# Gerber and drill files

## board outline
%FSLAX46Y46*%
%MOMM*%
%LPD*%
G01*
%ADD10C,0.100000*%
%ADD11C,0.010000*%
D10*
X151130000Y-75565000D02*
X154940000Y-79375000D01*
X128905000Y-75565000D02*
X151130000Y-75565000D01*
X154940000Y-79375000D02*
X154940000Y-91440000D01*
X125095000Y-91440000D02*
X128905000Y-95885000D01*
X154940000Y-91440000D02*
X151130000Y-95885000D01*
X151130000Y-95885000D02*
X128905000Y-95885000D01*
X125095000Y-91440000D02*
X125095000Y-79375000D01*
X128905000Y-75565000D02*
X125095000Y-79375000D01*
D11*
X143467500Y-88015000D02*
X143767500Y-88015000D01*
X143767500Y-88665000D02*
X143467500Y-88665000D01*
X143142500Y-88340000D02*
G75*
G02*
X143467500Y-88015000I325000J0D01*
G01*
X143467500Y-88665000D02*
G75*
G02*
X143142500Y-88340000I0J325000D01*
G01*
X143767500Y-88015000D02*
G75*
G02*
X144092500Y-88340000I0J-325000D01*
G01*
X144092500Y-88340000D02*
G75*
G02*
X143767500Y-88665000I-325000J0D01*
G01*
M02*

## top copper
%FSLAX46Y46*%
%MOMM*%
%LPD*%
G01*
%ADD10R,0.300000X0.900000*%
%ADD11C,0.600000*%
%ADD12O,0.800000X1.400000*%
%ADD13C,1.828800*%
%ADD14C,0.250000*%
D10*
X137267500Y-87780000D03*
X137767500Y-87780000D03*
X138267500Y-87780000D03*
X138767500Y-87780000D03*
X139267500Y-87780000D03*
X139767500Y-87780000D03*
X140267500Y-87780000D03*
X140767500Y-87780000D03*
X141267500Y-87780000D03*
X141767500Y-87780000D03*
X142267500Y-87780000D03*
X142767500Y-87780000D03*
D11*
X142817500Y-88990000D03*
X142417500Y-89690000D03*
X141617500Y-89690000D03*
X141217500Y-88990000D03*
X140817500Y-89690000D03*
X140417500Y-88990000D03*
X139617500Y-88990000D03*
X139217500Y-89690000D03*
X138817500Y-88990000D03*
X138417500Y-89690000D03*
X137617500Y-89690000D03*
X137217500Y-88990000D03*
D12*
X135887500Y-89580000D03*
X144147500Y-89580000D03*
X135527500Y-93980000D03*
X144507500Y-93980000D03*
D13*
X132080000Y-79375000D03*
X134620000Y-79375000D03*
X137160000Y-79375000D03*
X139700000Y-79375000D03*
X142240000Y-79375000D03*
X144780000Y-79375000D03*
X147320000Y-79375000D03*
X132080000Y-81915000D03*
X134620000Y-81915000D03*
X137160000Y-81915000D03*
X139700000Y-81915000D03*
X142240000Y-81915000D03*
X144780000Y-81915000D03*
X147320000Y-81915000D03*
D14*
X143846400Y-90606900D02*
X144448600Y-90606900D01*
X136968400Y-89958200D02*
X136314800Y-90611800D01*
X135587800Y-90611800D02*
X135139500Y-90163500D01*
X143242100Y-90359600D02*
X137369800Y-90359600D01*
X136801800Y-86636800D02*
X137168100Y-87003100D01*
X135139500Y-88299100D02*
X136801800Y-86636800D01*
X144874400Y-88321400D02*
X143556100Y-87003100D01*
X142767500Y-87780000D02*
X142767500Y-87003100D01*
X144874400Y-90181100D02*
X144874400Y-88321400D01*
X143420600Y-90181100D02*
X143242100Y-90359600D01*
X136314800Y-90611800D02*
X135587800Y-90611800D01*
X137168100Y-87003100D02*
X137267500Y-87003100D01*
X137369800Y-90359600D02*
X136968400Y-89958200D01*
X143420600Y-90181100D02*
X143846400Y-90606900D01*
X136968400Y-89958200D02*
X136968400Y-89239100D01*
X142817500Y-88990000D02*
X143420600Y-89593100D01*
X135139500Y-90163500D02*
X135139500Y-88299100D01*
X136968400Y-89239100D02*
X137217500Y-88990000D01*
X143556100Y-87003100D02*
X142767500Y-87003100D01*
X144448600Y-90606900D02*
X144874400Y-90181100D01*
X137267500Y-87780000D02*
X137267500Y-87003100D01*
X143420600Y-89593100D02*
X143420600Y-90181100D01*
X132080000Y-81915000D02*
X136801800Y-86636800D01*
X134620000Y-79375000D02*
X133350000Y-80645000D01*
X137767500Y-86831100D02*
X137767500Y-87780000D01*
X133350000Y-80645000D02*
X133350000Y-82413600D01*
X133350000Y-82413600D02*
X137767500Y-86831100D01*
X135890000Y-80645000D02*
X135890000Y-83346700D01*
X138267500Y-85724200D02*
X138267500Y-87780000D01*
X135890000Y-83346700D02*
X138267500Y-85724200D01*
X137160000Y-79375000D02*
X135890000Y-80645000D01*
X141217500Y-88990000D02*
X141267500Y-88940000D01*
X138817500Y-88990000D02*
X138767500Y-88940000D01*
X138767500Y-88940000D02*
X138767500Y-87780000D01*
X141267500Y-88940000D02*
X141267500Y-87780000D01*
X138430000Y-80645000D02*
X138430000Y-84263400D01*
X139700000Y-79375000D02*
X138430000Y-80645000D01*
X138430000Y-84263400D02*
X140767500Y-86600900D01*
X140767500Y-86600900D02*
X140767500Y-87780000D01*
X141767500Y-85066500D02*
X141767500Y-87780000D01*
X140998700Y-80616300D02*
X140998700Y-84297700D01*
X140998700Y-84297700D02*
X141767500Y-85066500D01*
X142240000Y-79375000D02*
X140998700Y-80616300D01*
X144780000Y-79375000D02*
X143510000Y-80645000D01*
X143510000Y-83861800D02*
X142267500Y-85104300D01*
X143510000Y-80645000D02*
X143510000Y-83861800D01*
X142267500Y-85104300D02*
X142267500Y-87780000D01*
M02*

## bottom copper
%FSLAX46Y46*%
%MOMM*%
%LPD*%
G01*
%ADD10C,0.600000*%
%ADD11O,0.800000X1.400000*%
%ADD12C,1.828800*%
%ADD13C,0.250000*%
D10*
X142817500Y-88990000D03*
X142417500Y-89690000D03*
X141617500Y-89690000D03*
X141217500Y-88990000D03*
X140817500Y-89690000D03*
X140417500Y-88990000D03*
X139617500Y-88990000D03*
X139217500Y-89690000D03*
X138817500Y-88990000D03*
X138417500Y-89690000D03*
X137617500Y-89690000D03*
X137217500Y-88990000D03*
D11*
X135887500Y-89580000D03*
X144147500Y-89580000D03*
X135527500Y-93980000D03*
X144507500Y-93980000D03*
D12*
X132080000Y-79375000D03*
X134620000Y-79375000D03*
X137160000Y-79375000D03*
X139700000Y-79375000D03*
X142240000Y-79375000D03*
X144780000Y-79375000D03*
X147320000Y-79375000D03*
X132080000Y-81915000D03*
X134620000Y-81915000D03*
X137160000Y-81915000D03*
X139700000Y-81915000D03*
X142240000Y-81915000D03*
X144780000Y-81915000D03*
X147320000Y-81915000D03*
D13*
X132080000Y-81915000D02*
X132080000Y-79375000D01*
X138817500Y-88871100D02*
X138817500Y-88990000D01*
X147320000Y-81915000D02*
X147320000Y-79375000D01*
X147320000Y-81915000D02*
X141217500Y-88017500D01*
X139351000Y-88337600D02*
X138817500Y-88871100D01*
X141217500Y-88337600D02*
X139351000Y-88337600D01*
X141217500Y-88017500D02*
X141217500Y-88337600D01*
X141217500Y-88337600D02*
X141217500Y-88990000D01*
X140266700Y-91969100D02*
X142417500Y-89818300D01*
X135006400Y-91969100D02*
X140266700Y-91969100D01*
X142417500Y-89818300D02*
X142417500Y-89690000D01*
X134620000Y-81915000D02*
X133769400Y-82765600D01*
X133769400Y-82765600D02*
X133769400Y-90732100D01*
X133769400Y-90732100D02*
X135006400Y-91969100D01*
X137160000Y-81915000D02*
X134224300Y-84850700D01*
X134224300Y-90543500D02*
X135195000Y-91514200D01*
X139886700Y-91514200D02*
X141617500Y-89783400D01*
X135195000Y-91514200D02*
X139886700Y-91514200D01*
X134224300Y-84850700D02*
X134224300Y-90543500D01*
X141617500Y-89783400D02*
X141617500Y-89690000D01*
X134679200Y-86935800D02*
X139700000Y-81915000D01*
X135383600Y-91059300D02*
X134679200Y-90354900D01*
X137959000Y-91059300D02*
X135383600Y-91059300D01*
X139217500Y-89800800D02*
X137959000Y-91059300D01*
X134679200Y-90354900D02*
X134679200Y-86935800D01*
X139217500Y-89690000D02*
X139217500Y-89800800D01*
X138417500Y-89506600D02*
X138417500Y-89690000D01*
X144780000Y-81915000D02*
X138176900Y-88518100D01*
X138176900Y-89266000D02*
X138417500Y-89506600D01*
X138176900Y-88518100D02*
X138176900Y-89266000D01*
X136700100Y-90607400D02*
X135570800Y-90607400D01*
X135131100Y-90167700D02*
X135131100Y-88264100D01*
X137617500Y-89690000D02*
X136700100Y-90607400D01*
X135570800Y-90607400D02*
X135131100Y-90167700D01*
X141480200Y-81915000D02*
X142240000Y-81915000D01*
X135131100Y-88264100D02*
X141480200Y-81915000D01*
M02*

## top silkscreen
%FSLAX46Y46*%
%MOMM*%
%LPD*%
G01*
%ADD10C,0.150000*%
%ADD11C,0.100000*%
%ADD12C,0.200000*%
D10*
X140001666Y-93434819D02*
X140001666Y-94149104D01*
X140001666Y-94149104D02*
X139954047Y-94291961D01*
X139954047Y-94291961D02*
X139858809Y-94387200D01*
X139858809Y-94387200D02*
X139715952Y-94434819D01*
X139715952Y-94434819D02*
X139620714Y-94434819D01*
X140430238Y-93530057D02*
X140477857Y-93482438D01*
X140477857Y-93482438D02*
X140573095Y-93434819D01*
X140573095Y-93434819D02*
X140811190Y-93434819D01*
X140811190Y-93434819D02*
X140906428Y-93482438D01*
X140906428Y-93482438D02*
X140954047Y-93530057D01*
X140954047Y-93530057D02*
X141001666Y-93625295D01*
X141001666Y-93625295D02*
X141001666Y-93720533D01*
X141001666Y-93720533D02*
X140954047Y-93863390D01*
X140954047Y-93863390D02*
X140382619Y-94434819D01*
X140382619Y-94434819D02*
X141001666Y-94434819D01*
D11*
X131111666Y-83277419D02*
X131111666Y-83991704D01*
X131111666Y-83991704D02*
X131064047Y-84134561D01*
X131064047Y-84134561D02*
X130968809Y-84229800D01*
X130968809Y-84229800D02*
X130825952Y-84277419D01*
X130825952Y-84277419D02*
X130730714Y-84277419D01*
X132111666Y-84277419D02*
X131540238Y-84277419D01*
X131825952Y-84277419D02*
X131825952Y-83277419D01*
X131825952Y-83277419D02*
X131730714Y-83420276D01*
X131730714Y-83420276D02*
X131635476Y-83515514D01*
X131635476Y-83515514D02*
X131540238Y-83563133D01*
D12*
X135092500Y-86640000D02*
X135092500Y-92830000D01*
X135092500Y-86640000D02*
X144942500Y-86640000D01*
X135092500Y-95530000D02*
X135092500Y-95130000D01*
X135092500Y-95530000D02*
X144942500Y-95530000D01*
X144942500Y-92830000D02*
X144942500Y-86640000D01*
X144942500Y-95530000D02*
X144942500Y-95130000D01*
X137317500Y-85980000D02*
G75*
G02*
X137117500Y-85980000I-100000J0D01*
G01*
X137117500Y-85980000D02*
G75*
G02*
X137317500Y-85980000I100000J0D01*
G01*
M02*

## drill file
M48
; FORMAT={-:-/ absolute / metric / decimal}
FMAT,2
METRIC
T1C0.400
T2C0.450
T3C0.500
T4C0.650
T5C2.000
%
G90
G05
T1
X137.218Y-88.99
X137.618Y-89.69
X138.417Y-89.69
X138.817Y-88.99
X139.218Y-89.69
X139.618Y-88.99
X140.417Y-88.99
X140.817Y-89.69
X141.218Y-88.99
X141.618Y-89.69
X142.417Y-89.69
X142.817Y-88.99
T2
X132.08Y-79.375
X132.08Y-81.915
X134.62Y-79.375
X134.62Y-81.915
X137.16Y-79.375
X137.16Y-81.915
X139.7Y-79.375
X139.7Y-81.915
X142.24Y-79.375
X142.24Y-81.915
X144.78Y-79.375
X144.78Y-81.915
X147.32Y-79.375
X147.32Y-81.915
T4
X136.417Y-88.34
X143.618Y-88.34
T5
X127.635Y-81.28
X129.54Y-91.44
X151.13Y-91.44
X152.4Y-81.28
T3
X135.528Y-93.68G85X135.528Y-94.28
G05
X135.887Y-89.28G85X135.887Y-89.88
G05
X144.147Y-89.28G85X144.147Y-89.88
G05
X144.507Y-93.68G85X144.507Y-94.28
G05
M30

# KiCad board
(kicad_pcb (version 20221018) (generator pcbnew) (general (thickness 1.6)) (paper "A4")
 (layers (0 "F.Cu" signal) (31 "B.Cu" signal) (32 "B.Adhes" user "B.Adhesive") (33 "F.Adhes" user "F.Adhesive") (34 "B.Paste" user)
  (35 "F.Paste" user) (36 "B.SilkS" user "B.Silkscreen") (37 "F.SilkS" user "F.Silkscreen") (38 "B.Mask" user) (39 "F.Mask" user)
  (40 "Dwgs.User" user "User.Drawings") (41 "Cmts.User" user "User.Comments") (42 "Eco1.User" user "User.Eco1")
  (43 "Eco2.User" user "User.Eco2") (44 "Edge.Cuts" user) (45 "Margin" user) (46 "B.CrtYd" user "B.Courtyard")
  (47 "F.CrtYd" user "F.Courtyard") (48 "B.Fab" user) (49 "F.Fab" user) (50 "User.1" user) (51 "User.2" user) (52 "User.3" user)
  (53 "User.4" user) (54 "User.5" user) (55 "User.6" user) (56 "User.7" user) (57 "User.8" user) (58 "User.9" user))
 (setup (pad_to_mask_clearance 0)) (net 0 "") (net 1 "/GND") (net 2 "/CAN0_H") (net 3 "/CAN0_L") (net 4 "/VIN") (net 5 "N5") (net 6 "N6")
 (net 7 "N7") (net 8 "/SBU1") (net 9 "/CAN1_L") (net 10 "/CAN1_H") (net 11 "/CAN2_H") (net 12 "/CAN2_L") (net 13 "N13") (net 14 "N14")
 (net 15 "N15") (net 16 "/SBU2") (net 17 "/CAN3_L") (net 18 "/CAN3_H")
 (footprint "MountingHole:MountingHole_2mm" (layer "F.Cu") (at 152.4 81.28)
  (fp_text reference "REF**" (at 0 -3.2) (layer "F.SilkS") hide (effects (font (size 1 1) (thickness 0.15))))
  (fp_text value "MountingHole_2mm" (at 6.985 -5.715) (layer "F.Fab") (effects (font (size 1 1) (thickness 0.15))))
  (pad "" np_thru_hole circle (at 0 0) (size 2 2) (drill 2) (layers "*.Cu" "*.Mask")))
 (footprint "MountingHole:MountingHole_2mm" (layer "F.Cu") (at 151.13 91.44)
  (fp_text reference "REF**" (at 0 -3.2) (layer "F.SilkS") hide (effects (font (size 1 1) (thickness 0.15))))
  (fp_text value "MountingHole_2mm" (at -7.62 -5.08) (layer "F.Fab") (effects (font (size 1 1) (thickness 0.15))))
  (pad "" np_thru_hole circle (at 0 0) (size 2 2) (drill 2) (layers "F&B.Cu" "*.Mask")))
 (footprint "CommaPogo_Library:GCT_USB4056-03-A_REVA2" (layer "F.Cu") (at 140.0175 93.98)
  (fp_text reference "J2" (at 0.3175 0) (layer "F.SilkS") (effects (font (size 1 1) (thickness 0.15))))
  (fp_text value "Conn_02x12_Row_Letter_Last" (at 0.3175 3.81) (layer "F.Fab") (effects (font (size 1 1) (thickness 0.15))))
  (fp_line (start -4.925 -7.34) (end -4.925 -1.15) (stroke (width 0.2) (type solid)) (layer "F.SilkS"))
  (fp_line (start -4.925 -7.34) (end 4.925 -7.34) (stroke (width 0.2) (type solid)) (layer "F.SilkS"))
  (fp_line (start -4.925 1.55) (end -4.925 1.15) (stroke (width 0.2) (type solid)) (layer "F.SilkS"))
  (fp_line (start -4.925 1.55) (end 4.925 1.55) (stroke (width 0.2) (type solid)) (layer "F.SilkS"))
  (fp_line (start 4.925 -1.15) (end 4.925 -7.34) (stroke (width 0.2) (type solid)) (layer "F.SilkS"))
  (fp_line (start 4.925 1.55) (end 4.925 1.15) (stroke (width 0.2) (type solid)) (layer "F.SilkS"))
  (fp_circle (center -2.8 -8) (end -2.7 -8) (stroke (width 0.2) (type solid)) (fill none) (layer "F.SilkS"))
  (fp_line (start 3.45 -5.965) (end 3.75 -5.965) (stroke (width 0.01) (type solid)) (layer "Edge.Cuts"))
  (fp_line (start 3.75 -5.315) (end 3.45 -5.315) (stroke (width 0.01) (type solid)) (layer "Edge.Cuts"))
  (fp_arc (start 3.125 -5.64) (mid 3.22019 -5.86981) (end 3.45 -5.965) (stroke (width 0.01) (type solid)) (layer "Edge.Cuts"))
  (fp_arc (start 3.45 -5.315) (mid 3.22019 -5.41019) (end 3.125 -5.64) (stroke (width 0.01) (type solid)) (layer "Edge.Cuts"))
  (fp_arc (start 3.75 -5.965) (mid 3.97981 -5.86981) (end 4.075 -5.64) (stroke (width 0.01) (type solid)) (layer "Edge.Cuts"))
  (fp_arc (start 4.075 -5.64) (mid 3.97981 -5.41019) (end 3.75 -5.315) (stroke (width 0.01) (type solid)) (layer "Edge.Cuts"))
  (pad "" np_thru_hole circle (at -3.6 -5.64) (size 0.65 0.65) (drill 0.65) (layers "*.Cu" "*.Mask"))
  (pad "" np_thru_hole circle (at 3.6 -5.64) (size 0.65 0.65) (drill 0.65) (layers "*.Cu" "*.Mask"))
  (pad "A1" smd rect (at -2.75 -6.2) (size 0.3 0.9) (layers "F.Cu" "F.Paste" "F.Mask") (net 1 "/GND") (solder_mask_margin 0.102))
  (pad "A2" smd rect (at -2.25 -6.2) (size 0.3 0.9) (layers "F.Cu" "F.Paste" "F.Mask") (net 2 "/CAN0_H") (solder_mask_margin 0.102))
  (pad "A3" smd rect (at -1.75 -6.2) (size 0.3 0.9) (layers "F.Cu" "F.Paste" "F.Mask") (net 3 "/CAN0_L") (solder_mask_margin 0.102))
  (pad "A4" smd rect (at -1.25 -6.2) (size 0.3 0.9) (layers "F.Cu" "F.Paste" "F.Mask") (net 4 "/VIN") (solder_mask_margin 0.102))
  (pad "A5" smd rect (at -0.75 -6.2) (size 0.3 0.9) (layers "F.Cu" "F.Paste" "F.Mask") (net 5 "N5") (solder_mask_margin 0.102))
  (pad "A6" smd rect (at -0.25 -6.2) (size 0.3 0.9) (layers "F.Cu" "F.Paste" "F.Mask") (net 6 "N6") (solder_mask_margin 0.102))
  (pad "A7" smd rect (at 0.25 -6.2) (size 0.3 0.9) (layers "F.Cu" "F.Paste" "F.Mask") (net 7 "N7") (solder_mask_margin 0.102))
  (pad "A8" smd rect (at 0.75 -6.2) (size 0.3 0.9) (layers "F.Cu" "F.Paste" "F.Mask") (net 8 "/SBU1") (solder_mask_margin 0.102))
  (pad "A9" smd rect (at 1.25 -6.2) (size 0.3 0.9) (layers "F.Cu" "F.Paste" "F.Mask") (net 4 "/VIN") (solder_mask_margin 0.102))
  (pad "A10" smd rect (at 1.75 -6.2) (size 0.3 0.9) (layers "F.Cu" "F.Paste" "F.Mask") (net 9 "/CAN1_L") (solder_mask_margin 0.102))
  (pad "A11" smd rect (at 2.25 -6.2) (size 0.3 0.9) (layers "F.Cu" "F.Paste" "F.Mask") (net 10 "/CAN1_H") (solder_mask_margin 0.102))
  (pad "A12" smd rect (at 2.75 -6.2) (size 0.3 0.9) (layers "F.Cu" "F.Paste" "F.Mask") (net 1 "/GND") (solder_mask_margin 0.102))
  (pad "B1" thru_hole circle (at 2.8 -4.99) (size 0.6 0.6) (drill 0.4) (layers "*.Cu" "*.Mask") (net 1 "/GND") (solder_mask_margin 0.102))
  (pad "B2" thru_hole circle (at 2.4 -4.29) (size 0.6 0.6) (drill 0.4) (layers "*.Cu" "*.Mask") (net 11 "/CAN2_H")
   (solder_mask_margin 0.102))
  (pad "B3" thru_hole circle (at 1.6 -4.29) (size 0.6 0.6) (drill 0.4) (layers "*.Cu" "*.Mask") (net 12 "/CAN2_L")
   (solder_mask_margin 0.102))
  (pad "B4" thru_hole circle (at 1.2 -4.99) (size 0.6 0.6) (drill 0.4) (layers "*.Cu" "*.Mask") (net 4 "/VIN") (solder_mask_margin 0.102))
  (pad "B5" thru_hole circle (at 0.8 -4.29) (size 0.6 0.6) (drill 0.4) (layers "*.Cu" "*.Mask") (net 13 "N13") (solder_mask_margin 0.102))
  (pad "B6" thru_hole circle (at 0.4 -4.99) (size 0.6 0.6) (drill 0.4) (layers "*.Cu" "*.Mask") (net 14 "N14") (solder_mask_margin 0.102))
  (pad "B7" thru_hole circle (at -0.4 -4.99) (size 0.6 0.6) (drill 0.4) (layers "*.Cu" "*.Mask") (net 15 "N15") (solder_mask_margin 0.102))
  (pad "B8" thru_hole circle (at -0.8 -4.29) (size 0.6 0.6) (drill 0.4) (layers "*.Cu" "*.Mask") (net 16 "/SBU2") (solder_mask_margin 0.102))
  (pad "B9" thru_hole circle (at -1.2 -4.99) (size 0.6 0.6) (drill 0.4) (layers "*.Cu" "*.Mask") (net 4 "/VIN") (solder_mask_margin 0.102))
  (pad "B10" thru_hole circle (at -1.6 -4.29) (size 0.6 0.6) (drill 0.4) (layers "*.Cu" "*.Mask") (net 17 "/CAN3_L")
   (solder_mask_margin 0.102))
  (pad "B11" thru_hole circle (at -2.4 -4.29) (size 0.6 0.6) (drill 0.4) (layers "*.Cu" "*.Mask") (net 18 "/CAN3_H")
   (solder_mask_margin 0.102))
  (pad "B12" thru_hole circle (at -2.8 -4.99) (size 0.6 0.6) (drill 0.4) (layers "*.Cu" "*.Mask") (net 1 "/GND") (solder_mask_margin 0.102))
  (pad "S1" thru_hole oval (at -4.13 -4.4) (size 0.8 1.4) (drill oval 0.5 1.1) (layers "*.Cu" "*.Mask") (solder_mask_margin 0.102))
  (pad "S2" thru_hole oval (at 4.13 -4.4) (size 0.8 1.4) (drill oval 0.5 1.1) (layers "*.Cu" "*.Mask") (solder_mask_margin 0.102))
  (pad "S3" thru_hole oval (at -4.49 0) (size 0.8 1.4) (drill oval 0.5 1.1) (layers "*.Cu" "*.Mask") (solder_mask_margin 0.102))
  (pad "S4" thru_hole oval (at 4.49 0) (size 0.8 1.4) (drill oval 0.5 1.1) (layers "*.Cu" "*.Mask") (solder_mask_margin 0.102)))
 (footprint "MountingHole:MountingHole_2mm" (layer "F.Cu") (at 127.635 81.28)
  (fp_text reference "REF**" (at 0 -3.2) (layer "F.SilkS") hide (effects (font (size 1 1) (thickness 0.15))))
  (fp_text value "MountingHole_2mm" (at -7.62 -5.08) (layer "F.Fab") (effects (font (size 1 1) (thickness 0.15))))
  (pad "" np_thru_hole circle (at 0 0) (size 2 2) (drill 2) (layers "*.Cu" "*.Mask")))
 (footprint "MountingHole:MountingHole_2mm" (layer "F.Cu") (at 129.54 91.44)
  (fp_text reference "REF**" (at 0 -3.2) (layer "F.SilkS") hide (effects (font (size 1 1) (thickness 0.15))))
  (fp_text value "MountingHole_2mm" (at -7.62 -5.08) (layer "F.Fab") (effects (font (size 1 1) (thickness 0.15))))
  (pad "" np_thru_hole circle (at 0 0) (size 2 2) (drill 2) (layers "F&B.Cu" "*.Mask")))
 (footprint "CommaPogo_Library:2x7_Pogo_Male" (layer "F.Cu") (at 139.7 83.82)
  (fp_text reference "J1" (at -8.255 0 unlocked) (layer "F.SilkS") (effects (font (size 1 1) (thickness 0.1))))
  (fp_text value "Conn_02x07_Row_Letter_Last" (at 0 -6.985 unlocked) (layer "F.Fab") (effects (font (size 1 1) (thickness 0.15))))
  (pad "1" thru_hole circle (at -7.62 -4.445) (size 1.8288 1.8288) (drill 0.45) (layers "*.Cu" "*.Mask") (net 1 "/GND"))
  (pad "2" thru_hole circle (at -5.08 -4.445) (size 1.8288 1.8288) (drill 0.45) (layers "*.Cu" "*.Mask") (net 2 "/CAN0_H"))
  (pad "3" thru_hole circle (at -2.54 -4.445) (size 1.8288 1.8288) (drill 0.45) (layers "*.Cu" "*.Mask") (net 3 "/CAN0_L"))
  (pad "4" thru_hole circle (at 0 -4.445) (size 1.8288 1.8288) (drill 0.45) (layers "*.Cu" "*.Mask") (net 8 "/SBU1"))
  (pad "5" thru_hole circle (at 2.54 -4.445) (size 1.8288 1.8288) (drill 0.45) (layers "*.Cu" "*.Mask") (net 9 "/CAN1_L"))
  (pad "6" thru_hole circle (at 5.08 -4.445) (size 1.8288 1.8288) (drill 0.45) (layers "*.Cu" "*.Mask") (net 10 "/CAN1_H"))
  (pad "7" thru_hole circle (at 7.62 -4.445) (size 1.8288 1.8288) (drill 0.45) (layers "*.Cu" "*.Mask") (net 4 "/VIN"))
  (pad "8" thru_hole circle (at -7.62 -1.905) (size 1.8288 1.8288) (drill 0.45) (layers "*.Cu" "*.Mask") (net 1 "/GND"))
  (pad "9" thru_hole circle (at -5.08 -1.905) (size 1.8288 1.8288) (drill 0.45) (layers "*.Cu" "*.Mask") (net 11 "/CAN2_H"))
  (pad "10" thru_hole circle (at -2.54 -1.905) (size 1.8288 1.8288) (drill 0.45) (layers "*.Cu" "*.Mask") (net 12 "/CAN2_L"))
  (pad "11" thru_hole circle (at 0 -1.905) (size 1.8288 1.8288) (drill 0.45) (layers "*.Cu" "*.Mask") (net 16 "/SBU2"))
  (pad "12" thru_hole circle (at 2.54 -1.905) (size 1.8288 1.8288) (drill 0.45) (layers "*.Cu" "*.Mask") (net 18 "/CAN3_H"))
  (pad "13" thru_hole circle (at 5.08 -1.905) (size 1.8288 1.8288) (drill 0.45) (layers "*.Cu" "*.Mask") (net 17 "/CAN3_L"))
  (pad "14" thru_hole circle (at 7.62 -1.905) (size 1.8288 1.8288) (drill 0.45) (layers "*.Cu" "*.Mask") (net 4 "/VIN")))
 (gr_line (start 151.13 75.565) (end 154.94 79.375) (stroke (width 0.1) (type default)) (layer "Edge.Cuts"))
 (gr_line (start 128.905 75.565) (end 151.13 75.565) (stroke (width 0.1) (type default)) (layer "Edge.Cuts"))
 (gr_line (start 154.94 79.375) (end 154.94 91.44) (stroke (width 0.1) (type default)) (layer "Edge.Cuts"))
 (gr_line (start 125.095 91.44) (end 128.905 95.885) (stroke (width 0.1) (type default)) (layer "Edge.Cuts"))
 (gr_line (start 154.94 91.44) (end 151.13 95.885) (stroke (width 0.1) (type default)) (layer "Edge.Cuts"))
 (gr_line (start 151.13 95.885) (end 128.905 95.885) (stroke (width 0.1) (type default)) (layer "Edge.Cuts"))
 (gr_line (start 125.095 91.44) (end 125.095 79.375) (stroke (width 0.1) (type default)) (layer "Edge.Cuts"))
 (gr_line (start 128.905 75.565) (end 125.095 79.375) (stroke (width 0.1) (type default)) (layer "Edge.Cuts"))
 (segment (start 143.8464 90.6069) (end 144.4486 90.6069) (width 0.25) (layer "F.Cu") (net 1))
 (segment (start 136.9684 89.9582) (end 136.3148 90.6118) (width 0.25) (layer "F.Cu") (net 1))
 (segment (start 135.5878 90.6118) (end 135.1395 90.1635) (width 0.25) (layer "F.Cu") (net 1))
 (segment (start 143.2421 90.3596) (end 137.3698 90.3596) (width 0.25) (layer "F.Cu") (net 1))
 (segment (start 136.8018 86.6368) (end 137.1681 87.0031) (width 0.25) (layer "F.Cu") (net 1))
 (segment (start 135.1395 88.2991) (end 136.8018 86.6368) (width 0.25) (layer "F.Cu") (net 1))
 (segment (start 144.8744 88.3214) (end 143.5561 87.0031) (width 0.25) (layer "F.Cu") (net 1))
 (segment (start 142.7675 87.78) (end 142.7675 87.0031) (width 0.25) (layer "F.Cu") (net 1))
 (segment (start 144.8744 90.1811) (end 144.8744 88.3214) (width 0.25) (layer "F.Cu") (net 1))
 (segment (start 143.4206 90.1811) (end 143.2421 90.3596) (width 0.25) (layer "F.Cu") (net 1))
 (segment (start 136.3148 90.6118) (end 135.5878 90.6118) (width 0.25) (layer "F.Cu") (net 1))
 (segment (start 137.1681 87.0031) (end 137.2675 87.0031) (width 0.25) (layer "F.Cu") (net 1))
 (segment (start 137.3698 90.3596) (end 136.9684 89.9582) (width 0.25) (layer "F.Cu") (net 1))
 (segment (start 143.4206 90.1811) (end 143.8464 90.6069) (width 0.25) (layer "F.Cu") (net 1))
 (segment (start 136.9684 89.9582) (end 136.9684 89.2391) (width 0.25) (layer "F.Cu") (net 1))
 (segment (start 142.8175 88.99) (end 143.4206 89.5931) (width 0.25) (layer "F.Cu") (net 1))
 (segment (start 135.1395 90.1635) (end 135.1395 88.2991) (width 0.25) (layer "F.Cu") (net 1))
 (segment (start 136.9684 89.2391) (end 137.2175 88.99) (width 0.25) (layer "F.Cu") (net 1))
 (segment (start 143.5561 87.0031) (end 142.7675 87.0031) (width 0.25) (layer "F.Cu") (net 1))
 (segment (start 144.4486 90.6069) (end 144.8744 90.1811) (width 0.25) (layer "F.Cu") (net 1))
 (segment (start 137.2675 87.78) (end 137.2675 87.0031) (width 0.25) (layer "F.Cu") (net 1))
 (segment (start 143.4206 89.5931) (end 143.4206 90.1811) (width 0.25) (layer "F.Cu") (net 1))
 (segment (start 132.08 81.915) (end 136.8018 86.6368) (width 0.25) (layer "F.Cu") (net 1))
 (segment (start 132.08 81.915) (end 132.08 79.375) (width 0.25) (layer "B.Cu") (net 1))
 (segment (start 134.62 79.375) (end 133.35 80.645) (width 0.25) (layer "F.Cu") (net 2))
 (segment (start 137.7675 86.8311) (end 137.7675 87.78) (width 0.25) (layer "F.Cu") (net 2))
 (segment (start 133.35 80.645) (end 133.35 82.4136) (width 0.25) (layer "F.Cu") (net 2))
 (segment (start 133.35 82.4136) (end 137.7675 86.8311) (width 0.25) (layer "F.Cu") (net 2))
 (segment (start 135.89 80.645) (end 135.89 83.3467) (width 0.25) (layer "F.Cu") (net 3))
 (segment (start 138.2675 85.7242) (end 138.2675 87.78) (width 0.25) (layer "F.Cu") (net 3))
 (segment (start 135.89 83.3467) (end 138.2675 85.7242) (width 0.25) (layer "F.Cu") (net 3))
 (segment (start 137.16 79.375) (end 135.89 80.645) (width 0.25) (layer "F.Cu") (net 3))
 (segment (start 141.2175 88.99) (end 141.2675 88.94) (width 0.25) (layer "F.Cu") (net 4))
 (segment (start 138.8175 88.99) (end 138.7675 88.94) (width 0.25) (layer "F.Cu") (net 4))
 (segment (start 138.7675 88.94) (end 138.7675 87.78) (width 0.25) (layer "F.Cu") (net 4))
 (segment (start 141.2675 88.94) (end 141.2675 87.78) (width 0.25) (layer "F.Cu") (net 4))
 (segment (start 138.8175 88.8711) (end 138.8175 88.99) (width 0.25) (layer "B.Cu") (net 4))
 (segment (start 147.32 81.915) (end 147.32 79.375) (width 0.25) (layer "B.Cu") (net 4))
 (segment (start 147.32 81.915) (end 141.2175 88.0175) (width 0.25) (layer "B.Cu") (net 4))
 (segment (start 139.351 88.3376) (end 138.8175 88.8711) (width 0.25) (layer "B.Cu") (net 4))
 (segment (start 141.2175 88.3376) (end 139.351 88.3376) (width 0.25) (layer "B.Cu") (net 4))
 (segment (start 141.2175 88.0175) (end 141.2175 88.3376) (width 0.25) (layer "B.Cu") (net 4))
 (segment (start 141.2175 88.3376) (end 141.2175 88.99) (width 0.25) (layer "B.Cu") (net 4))
 (segment (start 138.43 80.645) (end 138.43 84.2634) (width 0.25) (layer "F.Cu") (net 8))
 (segment (start 139.7 79.375) (end 138.43 80.645) (width 0.25) (layer "F.Cu") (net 8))
 (segment (start 138.43 84.2634) (end 140.7675 86.6009) (width 0.25) (layer "F.Cu") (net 8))
 (segment (start 140.7675 86.6009) (end 140.7675 87.78) (width 0.25) (layer "F.Cu") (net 8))
 (segment (start 141.7675 85.0665) (end 141.7675 87.78) (width 0.25) (layer "F.Cu") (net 9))
 (segment (start 140.9987 80.6163) (end 140.9987 84.2977) (width 0.25) (layer "F.Cu") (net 9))
 (segment (start 140.9987 84.2977) (end 141.7675 85.0665) (width 0.25) (layer "F.Cu") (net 9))
 (segment (start 142.24 79.375) (end 140.9987 80.6163) (width 0.25) (layer "F.Cu") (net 9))
 (segment (start 144.78 79.375) (end 143.51 80.645) (width 0.25) (layer "F.Cu") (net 10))
 (segment (start 143.51 83.8618) (end 142.2675 85.1043) (width 0.25) (layer "F.Cu") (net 10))
 (segment (start 143.51 80.645) (end 143.51 83.8618) (width 0.25) (layer "F.Cu") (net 10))
 (segment (start 142.2675 85.1043) (end 142.2675 87.78) (width 0.25) (layer "F.Cu") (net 10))
 (segment (start 140.2667 91.9691) (end 142.4175 89.8183) (width 0.25) (layer "B.Cu") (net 11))
 (segment (start 135.0064 91.9691) (end 140.2667 91.9691) (width 0.25) (layer "B.Cu") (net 11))
 (segment (start 142.4175 89.8183) (end 142.4175 89.69) (width 0.25) (layer "B.Cu") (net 11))
 (segment (start 134.62 81.915) (end 133.7694 82.7656) (width 0.25) (layer "B.Cu") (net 11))
 (segment (start 133.7694 82.7656) (end 133.7694 90.7321) (width 0.25) (layer "B.Cu") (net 11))
 (segment (start 133.7694 90.7321) (end 135.0064 91.9691) (width 0.25) (layer "B.Cu") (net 11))
 (segment (start 137.16 81.915) (end 134.2243 84.8507) (width 0.25) (layer "B.Cu") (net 12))
 (segment (start 134.2243 90.5435) (end 135.195 91.5142) (width 0.25) (layer "B.Cu") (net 12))
 (segment (start 139.8867 91.5142) (end 141.6175 89.7834) (width 0.25) (layer "B.Cu") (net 12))
 (segment (start 135.195 91.5142) (end 139.8867 91.5142) (width 0.25) (layer "B.Cu") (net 12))
 (segment (start 134.2243 84.8507) (end 134.2243 90.5435) (width 0.25) (layer "B.Cu") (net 12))
 (segment (start 141.6175 89.7834) (end 141.6175 89.69) (width 0.25) (layer "B.Cu") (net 12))
 (segment (start 134.6792 86.9358) (end 139.7 81.915) (width 0.25) (layer "B.Cu") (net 16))
 (segment (start 135.3836 91.0593) (end 134.6792 90.3549) (width 0.25) (layer "B.Cu") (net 16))
 (segment (start 137.959 91.0593) (end 135.3836 91.0593) (width 0.25) (layer "B.Cu") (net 16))
 (segment (start 139.2175 89.8008) (end 137.959 91.0593) (width 0.25) (layer "B.Cu") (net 16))
 (segment (start 134.6792 90.3549) (end 134.6792 86.9358) (width 0.25) (layer "B.Cu") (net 16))
 (segment (start 139.2175 89.69) (end 139.2175 89.8008) (width 0.25) (layer "B.Cu") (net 16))
 (segment (start 138.4175 89.5066) (end 138.4175 89.69) (width 0.25) (layer "B.Cu") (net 17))
 (segment (start 144.78 81.915) (end 138.1769 88.5181) (width 0.25) (layer "B.Cu") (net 17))
 (segment (start 138.1769 89.266) (end 138.4175 89.5066) (width 0.25) (layer "B.Cu") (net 17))
 (segment (start 138.1769 88.5181) (end 138.1769 89.266) (width 0.25) (layer "B.Cu") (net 17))
 (segment (start 136.7001 90.6074) (end 135.5708 90.6074) (width 0.25) (layer "B.Cu") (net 18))
 (segment (start 135.1311 90.1677) (end 135.1311 88.2641) (width 0.25) (layer "B.Cu") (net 18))
 (segment (start 137.6175 89.69) (end 136.7001 90.6074) (width 0.25) (layer "B.Cu") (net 18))
 (segment (start 135.5708 90.6074) (end 135.1311 90.1677) (width 0.25) (layer "B.Cu") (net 18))
 (segment (start 141.4802 81.915) (end 142.24 81.915) (width 0.25) (layer "B.Cu") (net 18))
 (segment (start 135.1311 88.2641) (end 141.4802 81.915) (width 0.25) (layer "B.Cu") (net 18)))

